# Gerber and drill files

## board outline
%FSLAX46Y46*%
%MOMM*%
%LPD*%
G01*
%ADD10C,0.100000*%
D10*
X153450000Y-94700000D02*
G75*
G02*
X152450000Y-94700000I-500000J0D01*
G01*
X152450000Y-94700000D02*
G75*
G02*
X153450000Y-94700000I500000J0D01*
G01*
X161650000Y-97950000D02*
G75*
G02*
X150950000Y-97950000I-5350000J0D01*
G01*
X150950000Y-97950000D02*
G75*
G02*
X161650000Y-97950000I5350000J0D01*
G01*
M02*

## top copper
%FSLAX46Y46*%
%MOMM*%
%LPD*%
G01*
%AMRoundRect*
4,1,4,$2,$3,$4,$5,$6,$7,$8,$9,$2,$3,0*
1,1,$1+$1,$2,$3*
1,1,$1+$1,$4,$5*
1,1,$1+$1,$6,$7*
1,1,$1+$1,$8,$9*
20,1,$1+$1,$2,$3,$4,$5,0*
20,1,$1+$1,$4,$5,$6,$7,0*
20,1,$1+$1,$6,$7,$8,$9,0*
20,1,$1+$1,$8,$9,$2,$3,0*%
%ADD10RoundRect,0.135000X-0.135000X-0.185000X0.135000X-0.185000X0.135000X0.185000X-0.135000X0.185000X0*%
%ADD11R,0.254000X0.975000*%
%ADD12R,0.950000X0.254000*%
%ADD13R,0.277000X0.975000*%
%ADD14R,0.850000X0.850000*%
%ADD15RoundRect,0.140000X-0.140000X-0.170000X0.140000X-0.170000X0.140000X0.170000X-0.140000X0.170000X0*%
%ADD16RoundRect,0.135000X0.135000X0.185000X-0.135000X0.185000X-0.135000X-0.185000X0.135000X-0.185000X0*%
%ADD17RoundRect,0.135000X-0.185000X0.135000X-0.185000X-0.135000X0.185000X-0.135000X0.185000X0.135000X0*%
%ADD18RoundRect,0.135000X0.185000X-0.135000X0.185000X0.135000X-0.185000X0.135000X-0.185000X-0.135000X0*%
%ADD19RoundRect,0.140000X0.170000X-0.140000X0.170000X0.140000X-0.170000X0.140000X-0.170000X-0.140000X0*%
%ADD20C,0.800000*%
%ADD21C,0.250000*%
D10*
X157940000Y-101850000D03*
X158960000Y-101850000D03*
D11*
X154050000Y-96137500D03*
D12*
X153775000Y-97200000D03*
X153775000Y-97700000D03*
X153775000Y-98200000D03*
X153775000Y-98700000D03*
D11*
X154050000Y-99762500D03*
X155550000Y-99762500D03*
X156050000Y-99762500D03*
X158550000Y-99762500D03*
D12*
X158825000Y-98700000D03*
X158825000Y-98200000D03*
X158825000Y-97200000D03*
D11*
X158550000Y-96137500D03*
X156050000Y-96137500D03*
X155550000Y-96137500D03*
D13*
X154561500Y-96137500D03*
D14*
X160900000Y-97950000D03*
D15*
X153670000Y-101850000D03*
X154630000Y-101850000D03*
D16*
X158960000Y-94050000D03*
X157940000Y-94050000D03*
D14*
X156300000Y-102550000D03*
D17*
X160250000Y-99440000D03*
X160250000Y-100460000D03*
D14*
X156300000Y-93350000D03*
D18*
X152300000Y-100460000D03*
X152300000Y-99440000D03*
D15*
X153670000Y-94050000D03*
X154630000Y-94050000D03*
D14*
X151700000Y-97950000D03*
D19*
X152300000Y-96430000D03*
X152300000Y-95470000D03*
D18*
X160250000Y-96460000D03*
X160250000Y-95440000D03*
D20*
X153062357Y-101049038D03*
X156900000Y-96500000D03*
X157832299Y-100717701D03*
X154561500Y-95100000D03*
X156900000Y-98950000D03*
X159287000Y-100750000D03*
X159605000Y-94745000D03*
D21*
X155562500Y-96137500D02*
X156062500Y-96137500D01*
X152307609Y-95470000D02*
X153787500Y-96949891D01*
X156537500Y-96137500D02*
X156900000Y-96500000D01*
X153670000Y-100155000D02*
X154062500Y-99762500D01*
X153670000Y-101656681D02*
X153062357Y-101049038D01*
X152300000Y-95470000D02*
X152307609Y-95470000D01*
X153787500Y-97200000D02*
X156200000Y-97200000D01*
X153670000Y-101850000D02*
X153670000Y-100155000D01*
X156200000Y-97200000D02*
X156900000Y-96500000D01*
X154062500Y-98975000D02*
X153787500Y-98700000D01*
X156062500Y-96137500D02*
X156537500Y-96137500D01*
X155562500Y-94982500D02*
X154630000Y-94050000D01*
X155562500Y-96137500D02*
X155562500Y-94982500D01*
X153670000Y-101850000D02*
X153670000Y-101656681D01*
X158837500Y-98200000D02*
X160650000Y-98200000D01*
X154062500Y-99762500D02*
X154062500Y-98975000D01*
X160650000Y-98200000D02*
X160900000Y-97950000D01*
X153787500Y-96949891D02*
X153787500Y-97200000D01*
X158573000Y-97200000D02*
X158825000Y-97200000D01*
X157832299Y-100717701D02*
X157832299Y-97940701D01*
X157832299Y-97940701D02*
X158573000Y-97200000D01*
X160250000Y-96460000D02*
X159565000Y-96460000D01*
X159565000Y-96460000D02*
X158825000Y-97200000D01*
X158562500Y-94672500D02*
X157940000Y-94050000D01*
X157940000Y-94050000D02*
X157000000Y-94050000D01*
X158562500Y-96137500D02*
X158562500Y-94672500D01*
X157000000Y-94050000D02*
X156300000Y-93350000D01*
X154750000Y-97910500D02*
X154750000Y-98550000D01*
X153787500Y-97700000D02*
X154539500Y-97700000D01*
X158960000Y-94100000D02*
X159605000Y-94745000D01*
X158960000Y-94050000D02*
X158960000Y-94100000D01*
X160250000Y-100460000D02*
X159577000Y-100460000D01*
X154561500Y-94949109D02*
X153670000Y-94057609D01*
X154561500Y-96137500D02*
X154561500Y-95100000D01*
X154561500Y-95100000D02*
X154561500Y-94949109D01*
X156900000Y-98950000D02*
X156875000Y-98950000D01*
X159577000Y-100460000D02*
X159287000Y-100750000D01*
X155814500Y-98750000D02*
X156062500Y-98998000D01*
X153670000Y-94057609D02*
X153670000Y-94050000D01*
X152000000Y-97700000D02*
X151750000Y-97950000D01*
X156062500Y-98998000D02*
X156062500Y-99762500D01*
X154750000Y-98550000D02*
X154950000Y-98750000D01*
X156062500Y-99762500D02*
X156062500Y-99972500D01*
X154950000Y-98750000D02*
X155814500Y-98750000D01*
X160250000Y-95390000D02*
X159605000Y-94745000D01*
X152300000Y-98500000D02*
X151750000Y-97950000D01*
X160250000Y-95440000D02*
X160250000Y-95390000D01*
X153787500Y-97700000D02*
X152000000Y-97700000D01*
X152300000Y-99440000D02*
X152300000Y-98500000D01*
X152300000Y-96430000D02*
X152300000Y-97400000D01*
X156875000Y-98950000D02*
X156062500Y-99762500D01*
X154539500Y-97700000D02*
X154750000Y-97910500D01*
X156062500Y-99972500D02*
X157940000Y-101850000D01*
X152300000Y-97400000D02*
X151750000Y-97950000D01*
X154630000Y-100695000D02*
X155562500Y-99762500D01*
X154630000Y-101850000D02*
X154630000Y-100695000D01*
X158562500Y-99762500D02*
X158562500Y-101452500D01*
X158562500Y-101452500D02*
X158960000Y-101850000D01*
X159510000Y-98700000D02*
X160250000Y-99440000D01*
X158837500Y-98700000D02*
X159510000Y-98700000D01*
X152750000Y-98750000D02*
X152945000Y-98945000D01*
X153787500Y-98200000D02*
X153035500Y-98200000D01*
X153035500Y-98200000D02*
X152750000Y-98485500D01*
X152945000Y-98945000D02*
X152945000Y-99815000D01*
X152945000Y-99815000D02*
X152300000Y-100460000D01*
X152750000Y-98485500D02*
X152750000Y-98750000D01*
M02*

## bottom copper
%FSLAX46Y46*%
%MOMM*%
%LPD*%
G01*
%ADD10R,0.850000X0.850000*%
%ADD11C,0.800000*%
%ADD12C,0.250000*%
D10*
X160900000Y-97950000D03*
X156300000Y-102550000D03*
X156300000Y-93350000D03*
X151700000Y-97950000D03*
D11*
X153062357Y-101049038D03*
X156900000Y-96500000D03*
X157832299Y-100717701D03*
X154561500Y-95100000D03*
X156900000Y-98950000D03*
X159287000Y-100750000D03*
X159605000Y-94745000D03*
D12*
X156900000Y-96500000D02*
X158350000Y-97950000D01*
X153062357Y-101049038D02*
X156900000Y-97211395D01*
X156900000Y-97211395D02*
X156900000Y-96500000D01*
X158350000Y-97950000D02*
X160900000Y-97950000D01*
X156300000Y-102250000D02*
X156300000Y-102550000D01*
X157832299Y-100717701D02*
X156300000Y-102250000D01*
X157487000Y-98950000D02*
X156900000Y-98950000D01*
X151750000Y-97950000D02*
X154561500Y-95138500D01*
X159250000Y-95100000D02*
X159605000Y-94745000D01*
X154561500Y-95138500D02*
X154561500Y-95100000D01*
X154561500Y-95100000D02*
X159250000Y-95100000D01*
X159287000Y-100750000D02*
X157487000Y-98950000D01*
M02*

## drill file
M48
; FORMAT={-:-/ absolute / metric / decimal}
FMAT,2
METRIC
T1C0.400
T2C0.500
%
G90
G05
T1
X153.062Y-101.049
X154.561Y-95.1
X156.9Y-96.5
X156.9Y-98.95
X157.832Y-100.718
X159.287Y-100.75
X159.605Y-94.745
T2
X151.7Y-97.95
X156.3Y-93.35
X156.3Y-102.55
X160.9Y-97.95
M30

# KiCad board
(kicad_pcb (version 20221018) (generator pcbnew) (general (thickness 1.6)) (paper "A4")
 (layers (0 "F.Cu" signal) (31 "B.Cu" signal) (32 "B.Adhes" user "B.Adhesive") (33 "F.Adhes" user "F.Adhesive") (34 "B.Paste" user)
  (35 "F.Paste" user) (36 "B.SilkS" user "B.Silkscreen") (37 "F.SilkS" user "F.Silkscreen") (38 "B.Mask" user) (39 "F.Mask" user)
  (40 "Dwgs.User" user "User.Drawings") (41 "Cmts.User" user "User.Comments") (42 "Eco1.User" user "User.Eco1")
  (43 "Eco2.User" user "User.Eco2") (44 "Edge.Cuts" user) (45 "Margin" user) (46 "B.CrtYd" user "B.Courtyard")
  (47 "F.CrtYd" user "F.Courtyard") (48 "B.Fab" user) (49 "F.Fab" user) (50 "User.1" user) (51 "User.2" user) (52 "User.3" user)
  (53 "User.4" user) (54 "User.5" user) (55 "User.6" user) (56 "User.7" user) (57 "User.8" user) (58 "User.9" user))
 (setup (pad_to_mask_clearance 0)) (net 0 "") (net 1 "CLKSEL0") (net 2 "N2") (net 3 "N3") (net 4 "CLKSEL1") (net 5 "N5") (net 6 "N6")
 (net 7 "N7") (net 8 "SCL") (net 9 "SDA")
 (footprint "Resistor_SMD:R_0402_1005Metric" (layer "F.Cu") (at 158.45 101.85)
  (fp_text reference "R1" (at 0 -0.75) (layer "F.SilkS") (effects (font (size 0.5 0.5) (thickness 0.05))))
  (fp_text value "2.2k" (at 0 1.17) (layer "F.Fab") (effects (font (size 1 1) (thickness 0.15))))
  (pad "1" smd roundrect (at -0.51 0) (size 0.54 0.64) (layers "F.Cu" "F.Paste" "F.Mask") (roundrect_rratio 0.25) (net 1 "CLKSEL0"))
  (pad "2" smd roundrect (at 0.51 0) (size 0.54 0.64) (layers "F.Cu" "F.Paste" "F.Mask") (roundrect_rratio 0.25) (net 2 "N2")))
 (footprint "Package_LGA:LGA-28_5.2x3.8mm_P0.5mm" (layer "F.Cu") (at 156.3 97.95)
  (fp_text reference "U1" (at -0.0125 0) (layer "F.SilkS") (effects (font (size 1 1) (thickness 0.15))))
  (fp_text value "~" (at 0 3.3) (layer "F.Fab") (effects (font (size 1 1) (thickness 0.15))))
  (pad "1" smd rect (at -2.25 -1.8125) (size 0.254 0.975) (layers "F.Cu" "F.Paste" "F.Mask") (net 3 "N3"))
  (pad "2" smd rect (at -2.525 -0.75 90) (size 0.254 0.95) (layers "F.Cu" "F.Paste" "F.Mask") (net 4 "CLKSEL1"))
  (pad "3" smd rect (at -2.525 -0.25 90) (size 0.254 0.95) (layers "F.Cu" "F.Paste" "F.Mask") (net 1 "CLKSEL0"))
  (pad "4" smd rect (at -2.525 0.25 90) (size 0.254 0.95) (layers "F.Cu" "F.Paste" "F.Mask") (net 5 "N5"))
  (pad "5" smd rect (at -2.525 0.75 90) (size 0.254 0.95) (layers "F.Cu" "F.Paste" "F.Mask") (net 4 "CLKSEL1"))
  (pad "6" smd rect (at -2.25 1.8125) (size 0.254 0.975) (layers "F.Cu" "F.Paste" "F.Mask") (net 4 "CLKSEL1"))
  (pad "9" smd rect (at -0.75 1.8125) (size 0.254 0.975) (layers "F.Cu" "F.Paste" "F.Mask") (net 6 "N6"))
  (pad "10" smd rect (at -0.25 1.8125) (size 0.254 0.975) (layers "F.Cu" "F.Paste" "F.Mask") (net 1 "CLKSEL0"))
  (pad "15" smd rect (at 2.25 1.8125) (size 0.254 0.975) (layers "F.Cu" "F.Paste" "F.Mask") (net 2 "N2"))
  (pad "16" smd rect (at 2.525 0.75 90) (size 0.254 0.95) (layers "F.Cu" "F.Paste" "F.Mask") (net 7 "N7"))
  (pad "17" smd rect (at 2.525 0.25 90) (size 0.254 0.95) (layers "F.Cu" "F.Paste" "F.Mask") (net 4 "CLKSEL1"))
  (pad "19" smd rect (at 2.525 -0.75 90) (size 0.254 0.95) (layers "F.Cu" "F.Paste" "F.Mask") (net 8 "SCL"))
  (pad "20" smd rect (at 2.25 -1.8125) (size 0.254 0.975) (layers "F.Cu" "F.Paste" "F.Mask") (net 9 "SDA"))
  (pad "25" smd rect (at -0.25 -1.8125) (size 0.254 0.975) (layers "F.Cu" "F.Paste" "F.Mask") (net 4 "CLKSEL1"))
  (pad "26" smd rect (at -0.75 -1.8125) (size 0.254 0.975) (layers "F.Cu" "F.Paste" "F.Mask") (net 4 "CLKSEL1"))
  (pad "28" smd rect (at -1.7385 -1.8125) (size 0.277 0.975) (layers "F.Cu" "F.Paste" "F.Mask") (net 1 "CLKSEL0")))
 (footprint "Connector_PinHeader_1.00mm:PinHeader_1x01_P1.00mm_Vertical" (layer "F.Cu") (at 160.9 97.95)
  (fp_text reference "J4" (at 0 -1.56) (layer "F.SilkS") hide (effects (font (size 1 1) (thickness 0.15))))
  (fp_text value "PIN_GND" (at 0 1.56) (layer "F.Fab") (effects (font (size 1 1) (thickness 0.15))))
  (pad "1" thru_hole rect (at 0 0) (size 0.85 0.85) (drill 0.5) (layers "*.Cu" "*.Mask") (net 4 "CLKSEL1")))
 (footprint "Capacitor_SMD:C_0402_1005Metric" (layer "F.Cu") (at 154.15 101.85)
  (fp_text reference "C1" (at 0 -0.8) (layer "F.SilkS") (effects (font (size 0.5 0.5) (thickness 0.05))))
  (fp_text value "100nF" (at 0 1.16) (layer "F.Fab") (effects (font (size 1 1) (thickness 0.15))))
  (pad "1" smd roundrect (at -0.48 0) (size 0.56 0.62) (layers "F.Cu" "F.Paste" "F.Mask") (roundrect_rratio 0.25) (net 4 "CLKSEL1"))
  (pad "2" smd roundrect (at 0.48 0) (size 0.56 0.62) (layers "F.Cu" "F.Paste" "F.Mask") (roundrect_rratio 0.25) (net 6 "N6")))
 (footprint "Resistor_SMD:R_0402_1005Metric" (layer "F.Cu") (at 158.45 94.05 180)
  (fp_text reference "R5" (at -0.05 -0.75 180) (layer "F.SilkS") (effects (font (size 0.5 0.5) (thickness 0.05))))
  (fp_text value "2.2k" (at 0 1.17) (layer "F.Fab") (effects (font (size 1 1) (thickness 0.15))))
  (pad "1" smd roundrect (at -0.51 0 180) (size 0.54 0.64) (layers "F.Cu" "F.Paste" "F.Mask") (roundrect_rratio 0.25) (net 1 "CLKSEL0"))
  (pad "2" smd roundrect (at 0.51 0 180) (size 0.54 0.64) (layers "F.Cu" "F.Paste" "F.Mask") (roundrect_rratio 0.25) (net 9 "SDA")))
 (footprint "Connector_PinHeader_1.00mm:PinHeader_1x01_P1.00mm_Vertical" (layer "F.Cu") (at 156.3 102.55)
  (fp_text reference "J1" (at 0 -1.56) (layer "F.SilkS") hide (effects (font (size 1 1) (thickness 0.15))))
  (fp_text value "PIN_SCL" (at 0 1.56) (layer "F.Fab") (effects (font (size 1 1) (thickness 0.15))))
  (pad "1" thru_hole rect (at 0 0) (size 0.85 0.85) (drill 0.5) (layers "*.Cu" "*.Mask") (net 8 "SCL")))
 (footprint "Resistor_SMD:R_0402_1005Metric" (layer "F.Cu") (at 160.25 99.95 -90)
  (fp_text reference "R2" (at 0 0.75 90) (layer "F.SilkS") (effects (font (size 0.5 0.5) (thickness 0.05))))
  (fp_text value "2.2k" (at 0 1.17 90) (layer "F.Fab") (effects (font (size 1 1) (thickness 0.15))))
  (pad "1" smd roundrect (at -0.51 0 270) (size 0.54 0.64) (layers "F.Cu" "F.Paste" "F.Mask") (roundrect_rratio 0.25) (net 7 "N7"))
  (pad "2" smd roundrect (at 0.51 0 270) (size 0.54 0.64) (layers "F.Cu" "F.Paste" "F.Mask") (roundrect_rratio 0.25) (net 1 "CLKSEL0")))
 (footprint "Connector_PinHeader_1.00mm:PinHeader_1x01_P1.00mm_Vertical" (layer "F.Cu") (at 156.3 93.35)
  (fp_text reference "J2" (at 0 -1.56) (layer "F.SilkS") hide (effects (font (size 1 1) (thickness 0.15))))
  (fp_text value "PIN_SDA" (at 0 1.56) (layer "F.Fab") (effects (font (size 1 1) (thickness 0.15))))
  (pad "1" thru_hole rect (at 0 0) (size 0.85 0.85) (drill 0.5) (layers "*.Cu" "*.Mask") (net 9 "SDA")))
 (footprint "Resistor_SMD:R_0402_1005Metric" (layer "F.Cu") (at 152.3 99.95 90)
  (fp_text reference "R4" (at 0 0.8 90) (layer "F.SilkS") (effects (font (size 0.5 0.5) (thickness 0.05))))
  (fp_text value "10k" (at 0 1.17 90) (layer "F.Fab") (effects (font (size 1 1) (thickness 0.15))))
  (pad "1" smd roundrect (at -0.51 0 90) (size 0.54 0.64) (layers "F.Cu" "F.Paste" "F.Mask") (roundrect_rratio 0.25) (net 5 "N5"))
  (pad "2" smd roundrect (at 0.51 0 90) (size 0.54 0.64) (layers "F.Cu" "F.Paste" "F.Mask") (roundrect_rratio 0.25) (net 1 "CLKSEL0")))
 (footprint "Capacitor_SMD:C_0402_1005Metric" (layer "F.Cu") (at 154.15 94.05)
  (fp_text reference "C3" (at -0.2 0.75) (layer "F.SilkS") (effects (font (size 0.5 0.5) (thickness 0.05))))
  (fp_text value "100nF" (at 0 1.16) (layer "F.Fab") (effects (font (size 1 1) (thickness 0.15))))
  (pad "1" smd roundrect (at -0.48 0) (size 0.56 0.62) (layers "F.Cu" "F.Paste" "F.Mask") (roundrect_rratio 0.25) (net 1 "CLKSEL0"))
  (pad "2" smd roundrect (at 0.48 0) (size 0.56 0.62) (layers "F.Cu" "F.Paste" "F.Mask") (roundrect_rratio 0.25) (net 4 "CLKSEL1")))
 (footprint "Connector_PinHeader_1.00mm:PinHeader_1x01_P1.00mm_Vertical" (layer "F.Cu") (at 151.7 97.95)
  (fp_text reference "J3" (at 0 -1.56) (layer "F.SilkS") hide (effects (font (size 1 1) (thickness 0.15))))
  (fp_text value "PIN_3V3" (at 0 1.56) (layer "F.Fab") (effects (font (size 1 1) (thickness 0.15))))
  (pad "1" thru_hole rect (at 0 0) (size 0.85 0.85) (drill 0.5) (layers "*.Cu" "*.Mask") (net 1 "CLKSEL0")))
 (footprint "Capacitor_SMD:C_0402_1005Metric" (layer "F.Cu") (at 152.3 95.95 90)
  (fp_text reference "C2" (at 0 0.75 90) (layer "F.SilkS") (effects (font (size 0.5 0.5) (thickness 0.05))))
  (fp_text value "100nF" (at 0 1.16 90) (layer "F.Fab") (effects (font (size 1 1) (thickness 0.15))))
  (pad "1" smd roundrect (at -0.48 0 90) (size 0.56 0.62) (layers "F.Cu" "F.Paste" "F.Mask") (roundrect_rratio 0.25) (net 1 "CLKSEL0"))
  (pad "2" smd roundrect (at 0.48 0 90) (size 0.56 0.62) (layers "F.Cu" "F.Paste" "F.Mask") (roundrect_rratio 0.25) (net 4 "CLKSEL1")))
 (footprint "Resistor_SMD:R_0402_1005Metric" (layer "F.Cu") (at 160.25 95.95 90)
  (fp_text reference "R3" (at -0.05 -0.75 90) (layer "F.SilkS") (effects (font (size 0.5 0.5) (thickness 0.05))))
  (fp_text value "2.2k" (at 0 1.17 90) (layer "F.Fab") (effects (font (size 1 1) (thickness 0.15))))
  (pad "1" smd roundrect (at -0.51 0 90) (size 0.54 0.64) (layers "F.Cu" "F.Paste" "F.Mask") (roundrect_rratio 0.25) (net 8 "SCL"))
  (pad "2" smd roundrect (at 0.51 0 90) (size 0.54 0.64) (layers "F.Cu" "F.Paste" "F.Mask") (roundrect_rratio 0.25) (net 1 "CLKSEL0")))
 (gr_circle (center 152.95 94.7) (end 153.45 94.7) (stroke (width 0.1) (type default)) (fill none) (layer "Edge.Cuts"))
 (gr_circle (center 156.3 97.95) (end 161.65 97.95) (stroke (width 0.1) (type default)) (fill none) (layer "Edge.Cuts"))
 (segment (start 155.5625 96.1375) (end 156.0625 96.1375) (width 0.25) (layer "F.Cu") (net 4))
 (segment (start 152.307609 95.47) (end 153.7875 96.949891) (width 0.25) (layer "F.Cu") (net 4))
 (segment (start 156.5375 96.1375) (end 156.9 96.5) (width 0.25) (layer "F.Cu") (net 4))
 (segment (start 153.67 100.155) (end 154.0625 99.7625) (width 0.25) (layer "F.Cu") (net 4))
 (segment (start 153.67 101.656681) (end 153.062357 101.049038) (width 0.25) (layer "F.Cu") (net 4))
 (segment (start 152.3 95.47) (end 152.307609 95.47) (width 0.25) (layer "F.Cu") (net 4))
 (segment (start 153.7875 97.2) (end 156.2 97.2) (width 0.25) (layer "F.Cu") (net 4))
 (segment (start 153.67 101.85) (end 153.67 100.155) (width 0.25) (layer "F.Cu") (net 4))
 (segment (start 156.2 97.2) (end 156.9 96.5) (width 0.25) (layer "F.Cu") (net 4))
 (segment (start 154.0625 98.975) (end 153.7875 98.7) (width 0.25) (layer "F.Cu") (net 4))
 (segment (start 156.0625 96.1375) (end 156.5375 96.1375) (width 0.25) (layer "F.Cu") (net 4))
 (segment (start 155.5625 94.9825) (end 154.63 94.05) (width 0.25) (layer "F.Cu") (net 4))
 (segment (start 155.5625 96.1375) (end 155.5625 94.9825) (width 0.25) (layer "F.Cu") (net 4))
 (segment (start 153.67 101.85) (end 153.67 101.656681) (width 0.25) (layer "F.Cu") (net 4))
 (segment (start 158.8375 98.2) (end 160.65 98.2) (width 0.25) (layer "F.Cu") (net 4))
 (segment (start 154.0625 99.7625) (end 154.0625 98.975) (width 0.25) (layer "F.Cu") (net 4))
 (segment (start 160.65 98.2) (end 160.9 97.95) (width 0.25) (layer "F.Cu") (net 4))
 (segment (start 153.7875 96.949891) (end 153.7875 97.2) (width 0.25) (layer "F.Cu") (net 4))
 (via (at 153.062357 101.049038) (size 0.8) (drill 0.4) (layers "F.Cu" "B.Cu") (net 4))
 (via (at 156.9 96.5) (size 0.8) (drill 0.4) (layers "F.Cu" "B.Cu") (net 4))
 (segment (start 156.9 96.5) (end 158.35 97.95) (width 0.25) (layer "B.Cu") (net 4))
 (segment (start 153.062357 101.049038) (end 156.9 97.211395) (width 0.25) (layer "B.Cu") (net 4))
 (segment (start 156.9 97.211395) (end 156.9 96.5) (width 0.25) (layer "B.Cu") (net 4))
 (segment (start 158.35 97.95) (end 160.9 97.95) (width 0.25) (layer "B.Cu") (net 4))
 (segment (start 158.573 97.2) (end 158.825 97.2) (width 0.25) (layer "F.Cu") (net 8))
 (segment (start 157.832299 100.717701) (end 157.832299 97.940701) (width 0.25) (layer "F.Cu") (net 8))
 (segment (start 157.832299 97.940701) (end 158.573 97.2) (width 0.25) (layer "F.Cu") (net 8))
 (segment (start 160.25 96.46) (end 159.565 96.46) (width 0.25) (layer "F.Cu") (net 8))
 (segment (start 159.565 96.46) (end 158.825 97.2) (width 0.25) (layer "F.Cu") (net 8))
 (via (at 157.832299 100.717701) (size 0.8) (drill 0.4) (layers "F.Cu" "B.Cu") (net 8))
 (segment (start 156.3 102.25) (end 156.3 102.55) (width 0.25) (layer "B.Cu") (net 8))
 (segment (start 157.832299 100.717701) (end 156.3 102.25) (width 0.25) (layer "B.Cu") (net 8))
 (segment (start 158.5625 94.6725) (end 157.94 94.05) (width 0.25) (layer "F.Cu") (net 9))
 (segment (start 157.94 94.05) (end 157 94.05) (width 0.25) (layer "F.Cu") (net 9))
 (segment (start 158.5625 96.1375) (end 158.5625 94.6725) (width 0.25) (layer "F.Cu") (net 9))
 (segment (start 157 94.05) (end 156.3 93.35) (width 0.25) (layer "F.Cu") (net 9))
 (segment (start 154.75 97.9105) (end 154.75 98.55) (width 0.25) (layer "F.Cu") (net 1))
 (segment (start 153.7875 97.7) (end 154.5395 97.7) (width 0.25) (layer "F.Cu") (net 1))
 (segment (start 158.96 94.1) (end 159.605 94.745) (width 0.25) (layer "F.Cu") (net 1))
 (segment (start 158.96 94.05) (end 158.96 94.1) (width 0.25) (layer "F.Cu") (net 1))
 (segment (start 160.25 100.46) (end 159.577 100.46) (width 0.25) (layer "F.Cu") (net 1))
 (segment (start 154.5615 94.949109) (end 153.67 94.057609) (width 0.25) (layer "F.Cu") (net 1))
 (segment (start 154.5615 96.1375) (end 154.5615 95.1) (width 0.25) (layer "F.Cu") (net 1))
 (segment (start 154.5615 95.1) (end 154.5615 94.949109) (width 0.25) (layer "F.Cu") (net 1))
 (segment (start 156.9 98.95) (end 156.875 98.95) (width 0.25) (layer "F.Cu") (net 1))
 (segment (start 159.577 100.46) (end 159.287 100.75) (width 0.25) (layer "F.Cu") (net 1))
 (segment (start 155.8145 98.75) (end 156.0625 98.998) (width 0.25) (layer "F.Cu") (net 1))
 (segment (start 153.67 94.057609) (end 153.67 94.05) (width 0.25) (layer "F.Cu") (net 1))
 (segment (start 152 97.7) (end 151.75 97.95) (width 0.25) (layer "F.Cu") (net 1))
 (segment (start 156.0625 98.998) (end 156.0625 99.7625) (width 0.25) (layer "F.Cu") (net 1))
 (segment (start 154.75 98.55) (end 154.95 98.75) (width 0.25) (layer "F.Cu") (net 1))
 (segment (start 156.0625 99.7625) (end 156.0625 99.9725) (width 0.25) (layer "F.Cu") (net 1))
 (segment (start 154.95 98.75) (end 155.8145 98.75) (width 0.25) (layer "F.Cu") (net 1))
 (segment (start 160.25 95.39) (end 159.605 94.745) (width 0.25) (layer "F.Cu") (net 1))
 (segment (start 152.3 98.5) (end 151.75 97.95) (width 0.25) (layer "F.Cu") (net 1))
 (segment (start 160.25 95.44) (end 160.25 95.39) (width 0.25) (layer "F.Cu") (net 1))
 (segment (start 153.7875 97.7) (end 152 97.7) (width 0.25) (layer "F.Cu") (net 1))
 (segment (start 152.3 99.44) (end 152.3 98.5) (width 0.25) (layer "F.Cu") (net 1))
 (segment (start 152.3 96.43) (end 152.3 97.4) (width 0.25) (layer "F.Cu") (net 1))
 (segment (start 156.875 98.95) (end 156.0625 99.7625) (width 0.25) (layer "F.Cu") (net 1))
 (segment (start 154.5395 97.7) (end 154.75 97.9105) (width 0.25) (layer "F.Cu") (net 1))
 (segment (start 156.0625 99.9725) (end 157.94 101.85) (width 0.25) (layer "F.Cu") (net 1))
 (segment (start 152.3 97.4) (end 151.75 97.95) (width 0.25) (layer "F.Cu") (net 1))
 (via (at 154.5615 95.1) (size 0.8) (drill 0.4) (layers "F.Cu" "B.Cu") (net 1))
 (via (at 156.9 98.95) (size 0.8) (drill 0.4) (layers "F.Cu" "B.Cu") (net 1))
 (via (at 159.287 100.75) (size 0.8) (drill 0.4) (layers "F.Cu" "B.Cu") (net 1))
 (via (at 159.605 94.745) (size 0.8) (drill 0.4) (layers "F.Cu" "B.Cu") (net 1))
 (segment (start 157.487 98.95) (end 156.9 98.95) (width 0.25) (layer "B.Cu") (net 1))
 (segment (start 151.75 97.95) (end 154.5615 95.1385) (width 0.25) (layer "B.Cu") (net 1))
 (segment (start 159.25 95.1) (end 159.605 94.745) (width 0.25) (layer "B.Cu") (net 1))
 (segment (start 154.5615 95.1385) (end 154.5615 95.1) (width 0.25) (layer "B.Cu") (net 1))
 (segment (start 154.5615 95.1) (end 159.25 95.1) (width 0.25) (layer "B.Cu") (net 1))
 (segment (start 159.287 100.75) (end 157.487 98.95) (width 0.25) (layer "B.Cu") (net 1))
 (segment (start 154.63 100.695) (end 155.5625 99.7625) (width 0.25) (layer "F.Cu") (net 6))
 (segment (start 154.63 101.85) (end 154.63 100.695) (width 0.25) (layer "F.Cu") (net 6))
 (segment (start 158.5625 99.7625) (end 158.5625 101.4525) (width 0.25) (layer "F.Cu") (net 2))
 (segment (start 158.5625 101.4525) (end 158.96 101.85) (width 0.25) (layer "F.Cu") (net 2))
 (segment (start 159.51 98.7) (end 160.25 99.44) (width 0.25) (layer "F.Cu") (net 7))
 (segment (start 158.8375 98.7) (end 159.51 98.7) (width 0.25) (layer "F.Cu") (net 7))
 (segment (start 152.75 98.75) (end 152.945 98.945) (width 0.25) (layer "F.Cu") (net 5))
 (segment (start 153.7875 98.2) (end 153.0355 98.2) (width 0.25) (layer "F.Cu") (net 5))
 (segment (start 153.0355 98.2) (end 152.75 98.4855) (width 0.25) (layer "F.Cu") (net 5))
 (segment (start 152.945 98.945) (end 152.945 99.815) (width 0.25) (layer "F.Cu") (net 5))
 (segment (start 152.945 99.815) (end 152.3 100.46) (width 0.25) (layer "F.Cu") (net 5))
 (segment (start 152.75 98.4855) (end 152.75 98.75) (width 0.25) (layer "F.Cu") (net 5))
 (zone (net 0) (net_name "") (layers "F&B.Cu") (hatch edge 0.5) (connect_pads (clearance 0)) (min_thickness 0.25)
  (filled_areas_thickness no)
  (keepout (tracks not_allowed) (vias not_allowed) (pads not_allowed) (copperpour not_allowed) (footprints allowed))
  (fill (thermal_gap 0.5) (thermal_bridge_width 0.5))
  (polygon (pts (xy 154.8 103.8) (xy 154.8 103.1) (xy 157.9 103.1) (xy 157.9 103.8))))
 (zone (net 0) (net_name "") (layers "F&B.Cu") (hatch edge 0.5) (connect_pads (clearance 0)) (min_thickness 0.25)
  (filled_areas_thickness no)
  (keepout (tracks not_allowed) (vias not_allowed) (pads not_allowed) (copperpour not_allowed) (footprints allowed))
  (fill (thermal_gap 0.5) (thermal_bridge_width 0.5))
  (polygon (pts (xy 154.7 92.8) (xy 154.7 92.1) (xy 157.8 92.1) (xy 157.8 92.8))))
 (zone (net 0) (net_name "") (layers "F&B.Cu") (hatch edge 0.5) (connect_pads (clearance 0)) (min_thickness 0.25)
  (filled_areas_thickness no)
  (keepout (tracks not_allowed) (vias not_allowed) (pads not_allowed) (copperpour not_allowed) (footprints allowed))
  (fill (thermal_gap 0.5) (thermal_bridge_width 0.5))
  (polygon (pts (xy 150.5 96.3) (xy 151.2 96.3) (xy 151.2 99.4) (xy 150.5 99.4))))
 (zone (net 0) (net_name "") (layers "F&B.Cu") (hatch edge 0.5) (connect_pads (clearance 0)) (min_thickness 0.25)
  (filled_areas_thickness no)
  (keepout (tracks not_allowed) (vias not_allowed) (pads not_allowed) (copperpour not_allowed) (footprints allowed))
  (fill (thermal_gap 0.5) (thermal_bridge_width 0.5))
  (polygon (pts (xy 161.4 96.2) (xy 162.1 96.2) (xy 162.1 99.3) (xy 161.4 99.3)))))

